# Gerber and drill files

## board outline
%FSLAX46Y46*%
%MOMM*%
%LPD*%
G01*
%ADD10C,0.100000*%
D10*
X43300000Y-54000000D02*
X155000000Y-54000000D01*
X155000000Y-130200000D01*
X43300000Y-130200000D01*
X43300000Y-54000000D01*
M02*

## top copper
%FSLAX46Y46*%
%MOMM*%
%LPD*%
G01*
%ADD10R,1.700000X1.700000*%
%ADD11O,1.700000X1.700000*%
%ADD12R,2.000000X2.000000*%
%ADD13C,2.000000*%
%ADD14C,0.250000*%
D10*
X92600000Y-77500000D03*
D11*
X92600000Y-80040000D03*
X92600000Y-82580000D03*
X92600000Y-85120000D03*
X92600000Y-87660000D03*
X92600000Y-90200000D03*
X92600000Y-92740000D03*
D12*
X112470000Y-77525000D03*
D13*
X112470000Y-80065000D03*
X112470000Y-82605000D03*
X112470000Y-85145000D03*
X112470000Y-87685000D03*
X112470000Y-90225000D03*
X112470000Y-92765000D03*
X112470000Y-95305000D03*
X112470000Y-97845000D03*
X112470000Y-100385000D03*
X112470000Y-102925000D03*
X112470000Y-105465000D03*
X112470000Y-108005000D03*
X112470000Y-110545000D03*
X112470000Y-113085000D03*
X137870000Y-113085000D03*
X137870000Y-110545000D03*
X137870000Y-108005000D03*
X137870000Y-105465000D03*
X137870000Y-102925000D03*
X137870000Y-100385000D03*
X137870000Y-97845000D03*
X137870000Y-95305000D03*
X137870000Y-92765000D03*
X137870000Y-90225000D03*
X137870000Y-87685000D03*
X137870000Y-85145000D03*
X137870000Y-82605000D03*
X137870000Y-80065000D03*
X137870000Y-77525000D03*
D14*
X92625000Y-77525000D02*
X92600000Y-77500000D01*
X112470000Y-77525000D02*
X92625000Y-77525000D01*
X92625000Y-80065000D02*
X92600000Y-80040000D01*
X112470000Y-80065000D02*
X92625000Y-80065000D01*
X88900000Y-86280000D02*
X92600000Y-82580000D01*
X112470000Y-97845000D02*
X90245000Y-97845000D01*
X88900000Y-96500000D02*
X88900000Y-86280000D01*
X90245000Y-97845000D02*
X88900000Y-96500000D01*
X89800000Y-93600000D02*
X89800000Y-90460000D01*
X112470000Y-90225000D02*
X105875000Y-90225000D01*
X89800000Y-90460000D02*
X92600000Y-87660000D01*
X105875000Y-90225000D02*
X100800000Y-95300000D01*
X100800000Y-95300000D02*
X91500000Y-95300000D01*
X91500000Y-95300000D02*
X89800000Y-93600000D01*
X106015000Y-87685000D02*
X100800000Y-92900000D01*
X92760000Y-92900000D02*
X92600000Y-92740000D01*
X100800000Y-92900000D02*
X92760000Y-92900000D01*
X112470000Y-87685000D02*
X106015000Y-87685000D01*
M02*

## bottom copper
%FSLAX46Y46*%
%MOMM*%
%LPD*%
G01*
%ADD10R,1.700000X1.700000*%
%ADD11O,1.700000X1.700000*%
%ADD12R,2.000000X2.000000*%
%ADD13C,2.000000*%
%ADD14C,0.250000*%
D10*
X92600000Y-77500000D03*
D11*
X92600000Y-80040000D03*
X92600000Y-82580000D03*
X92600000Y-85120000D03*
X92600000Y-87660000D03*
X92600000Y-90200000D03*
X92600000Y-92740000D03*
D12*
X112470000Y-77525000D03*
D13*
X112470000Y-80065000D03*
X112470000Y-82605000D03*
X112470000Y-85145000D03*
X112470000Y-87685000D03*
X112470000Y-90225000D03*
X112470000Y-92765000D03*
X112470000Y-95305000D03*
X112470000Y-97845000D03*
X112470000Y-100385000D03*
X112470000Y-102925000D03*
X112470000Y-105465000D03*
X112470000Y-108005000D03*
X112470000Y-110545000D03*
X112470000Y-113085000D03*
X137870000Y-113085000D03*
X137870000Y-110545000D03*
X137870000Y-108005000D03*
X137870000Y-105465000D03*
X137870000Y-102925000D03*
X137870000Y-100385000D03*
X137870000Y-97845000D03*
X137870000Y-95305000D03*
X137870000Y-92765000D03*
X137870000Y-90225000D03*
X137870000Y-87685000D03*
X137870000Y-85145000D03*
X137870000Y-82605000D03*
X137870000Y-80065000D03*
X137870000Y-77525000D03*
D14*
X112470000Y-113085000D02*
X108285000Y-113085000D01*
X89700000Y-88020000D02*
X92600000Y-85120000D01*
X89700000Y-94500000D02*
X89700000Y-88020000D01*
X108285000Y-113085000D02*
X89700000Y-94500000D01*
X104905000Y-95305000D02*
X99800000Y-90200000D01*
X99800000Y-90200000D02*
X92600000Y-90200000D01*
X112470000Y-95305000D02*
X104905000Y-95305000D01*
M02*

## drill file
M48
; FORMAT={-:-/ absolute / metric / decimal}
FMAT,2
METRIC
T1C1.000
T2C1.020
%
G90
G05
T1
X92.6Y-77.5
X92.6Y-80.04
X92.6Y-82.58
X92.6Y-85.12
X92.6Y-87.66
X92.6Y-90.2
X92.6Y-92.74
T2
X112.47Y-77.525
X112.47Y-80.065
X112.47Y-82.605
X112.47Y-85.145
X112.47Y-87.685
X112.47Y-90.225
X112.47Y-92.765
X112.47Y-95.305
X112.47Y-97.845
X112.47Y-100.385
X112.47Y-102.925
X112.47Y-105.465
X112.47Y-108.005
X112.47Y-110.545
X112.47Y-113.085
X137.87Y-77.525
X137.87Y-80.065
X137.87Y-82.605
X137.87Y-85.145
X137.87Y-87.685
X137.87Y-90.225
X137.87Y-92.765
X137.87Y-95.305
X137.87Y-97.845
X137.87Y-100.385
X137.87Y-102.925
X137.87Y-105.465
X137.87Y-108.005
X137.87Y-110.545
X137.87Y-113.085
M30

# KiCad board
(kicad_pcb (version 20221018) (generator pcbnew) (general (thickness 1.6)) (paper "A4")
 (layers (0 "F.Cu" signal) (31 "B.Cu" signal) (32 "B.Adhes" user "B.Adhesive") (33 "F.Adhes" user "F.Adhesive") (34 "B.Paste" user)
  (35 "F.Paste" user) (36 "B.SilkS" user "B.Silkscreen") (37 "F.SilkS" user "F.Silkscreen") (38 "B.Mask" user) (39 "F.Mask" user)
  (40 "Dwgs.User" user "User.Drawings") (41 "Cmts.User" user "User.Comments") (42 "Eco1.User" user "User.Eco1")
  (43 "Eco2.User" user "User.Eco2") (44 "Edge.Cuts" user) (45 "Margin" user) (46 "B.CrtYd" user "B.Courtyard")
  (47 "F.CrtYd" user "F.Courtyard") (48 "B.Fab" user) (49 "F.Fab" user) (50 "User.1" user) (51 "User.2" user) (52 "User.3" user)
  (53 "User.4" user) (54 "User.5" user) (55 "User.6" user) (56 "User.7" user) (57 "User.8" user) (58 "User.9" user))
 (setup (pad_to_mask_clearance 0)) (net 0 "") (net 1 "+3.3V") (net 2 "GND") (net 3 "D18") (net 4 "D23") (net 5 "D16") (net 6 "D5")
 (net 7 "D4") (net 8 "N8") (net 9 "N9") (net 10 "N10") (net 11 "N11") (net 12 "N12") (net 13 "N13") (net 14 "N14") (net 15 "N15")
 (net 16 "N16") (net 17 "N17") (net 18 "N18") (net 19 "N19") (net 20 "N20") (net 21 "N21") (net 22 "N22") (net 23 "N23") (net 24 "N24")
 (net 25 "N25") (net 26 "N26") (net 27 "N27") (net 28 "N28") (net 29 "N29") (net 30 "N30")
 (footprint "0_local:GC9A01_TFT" (layer "F.Cu") (at 92.6 77.5)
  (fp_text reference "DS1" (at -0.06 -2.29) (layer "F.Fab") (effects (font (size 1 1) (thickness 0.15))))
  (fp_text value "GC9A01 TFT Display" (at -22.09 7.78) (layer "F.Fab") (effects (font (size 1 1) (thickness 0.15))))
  (pad "1" thru_hole rect (at 0 0) (size 1.7 1.7) (drill 1) (layers "*.Cu" "*.Mask") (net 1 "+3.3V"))
  (pad "2" thru_hole oval (at 0 2.54) (size 1.7 1.7) (drill 1) (layers "*.Cu" "*.Mask") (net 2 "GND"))
  (pad "3" thru_hole oval (at 0 5.08) (size 1.7 1.7) (drill 1) (layers "*.Cu" "*.Mask") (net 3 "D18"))
  (pad "4" thru_hole oval (at 0 7.62) (size 1.7 1.7) (drill 1) (layers "*.Cu" "*.Mask") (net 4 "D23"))
  (pad "5" thru_hole oval (at 0 10.16) (size 1.7 1.7) (drill 1) (layers "*.Cu" "*.Mask") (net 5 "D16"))
  (pad "6" thru_hole oval (at 0 12.7) (size 1.7 1.7) (drill 1) (layers "*.Cu" "*.Mask") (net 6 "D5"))
  (pad "7" thru_hole oval (at 0 15.24) (size 1.7 1.7) (drill 1) (layers "*.Cu" "*.Mask") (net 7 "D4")))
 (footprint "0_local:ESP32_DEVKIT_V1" (layer "F.Cu") (at 125.17 93.04)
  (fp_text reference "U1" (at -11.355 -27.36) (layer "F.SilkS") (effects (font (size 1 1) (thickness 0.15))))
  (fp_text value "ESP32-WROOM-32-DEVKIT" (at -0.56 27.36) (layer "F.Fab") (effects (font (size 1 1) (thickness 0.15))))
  (pad "1" thru_hole rect (at -12.7 -15.515) (size 2 2) (drill 1.02) (layers "*.Cu" "*.Mask") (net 1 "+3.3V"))
  (pad "2" thru_hole circle (at -12.7 -12.975) (size 2 2) (drill 1.02) (layers "*.Cu" "*.Mask") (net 2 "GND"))
  (pad "3" thru_hole circle (at -12.7 -10.435) (size 2 2) (drill 1.02) (layers "*.Cu" "*.Mask") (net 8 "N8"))
  (pad "4" thru_hole circle (at -12.7 -7.895) (size 2 2) (drill 1.02) (layers "*.Cu" "*.Mask") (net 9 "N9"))
  (pad "5" thru_hole circle (at -12.7 -5.355) (size 2 2) (drill 1.02) (layers "*.Cu" "*.Mask") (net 7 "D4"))
  (pad "6" thru_hole circle (at -12.7 -2.815) (size 2 2) (drill 1.02) (layers "*.Cu" "*.Mask") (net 5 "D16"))
  (pad "7" thru_hole circle (at -12.7 -0.275) (size 2 2) (drill 1.02) (layers "*.Cu" "*.Mask") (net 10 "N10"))
  (pad "8" thru_hole circle (at -12.7 2.265) (size 2 2) (drill 1.02) (layers "*.Cu" "*.Mask") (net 6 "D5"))
  (pad "9" thru_hole circle (at -12.7 4.805) (size 2 2) (drill 1.02) (layers "*.Cu" "*.Mask") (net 3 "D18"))
  (pad "10" thru_hole circle (at -12.7 7.345) (size 2 2) (drill 1.02) (layers "*.Cu" "*.Mask") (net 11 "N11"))
  (pad "11" thru_hole circle (at -12.7 9.885) (size 2 2) (drill 1.02) (layers "*.Cu" "*.Mask") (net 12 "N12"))
  (pad "12" thru_hole circle (at -12.7 12.425) (size 2 2) (drill 1.02) (layers "*.Cu" "*.Mask") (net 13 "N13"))
  (pad "13" thru_hole circle (at -12.7 14.965) (size 2 2) (drill 1.02) (layers "*.Cu" "*.Mask") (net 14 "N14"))
  (pad "14" thru_hole circle (at -12.7 17.505) (size 2 2) (drill 1.02) (layers "*.Cu" "*.Mask") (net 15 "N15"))
  (pad "15" thru_hole circle (at -12.7 20.045) (size 2 2) (drill 1.02) (layers "*.Cu" "*.Mask") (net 4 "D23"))
  (pad "16" thru_hole circle (at 12.7 20.045) (size 2 2) (drill 1.02) (layers "*.Cu" "*.Mask") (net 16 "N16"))
  (pad "17" thru_hole circle (at 12.7 17.505) (size 2 2) (drill 1.02) (layers "*.Cu" "*.Mask") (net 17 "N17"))
  (pad "18" thru_hole circle (at 12.7 14.965) (size 2 2) (drill 1.02) (layers "*.Cu" "*.Mask") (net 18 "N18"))
  (pad "19" thru_hole circle (at 12.7 12.425) (size 2 2) (drill 1.02) (layers "*.Cu" "*.Mask") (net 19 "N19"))
  (pad "20" thru_hole circle (at 12.7 9.885) (size 2 2) (drill 1.02) (layers "*.Cu" "*.Mask") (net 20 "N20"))
  (pad "21" thru_hole circle (at 12.7 7.345) (size 2 2) (drill 1.02) (layers "*.Cu" "*.Mask") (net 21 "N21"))
  (pad "22" thru_hole circle (at 12.7 4.805) (size 2 2) (drill 1.02) (layers "*.Cu" "*.Mask") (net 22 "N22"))
  (pad "23" thru_hole circle (at 12.7 2.265) (size 2 2) (drill 1.02) (layers "*.Cu" "*.Mask") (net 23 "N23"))
  (pad "24" thru_hole circle (at 12.7 -0.275) (size 2 2) (drill 1.02) (layers "*.Cu" "*.Mask") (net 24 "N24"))
  (pad "25" thru_hole circle (at 12.7 -2.815) (size 2 2) (drill 1.02) (layers "*.Cu" "*.Mask") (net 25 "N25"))
  (pad "26" thru_hole circle (at 12.7 -5.355) (size 2 2) (drill 1.02) (layers "*.Cu" "*.Mask") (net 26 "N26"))
  (pad "27" thru_hole circle (at 12.7 -7.895) (size 2 2) (drill 1.02) (layers "*.Cu" "*.Mask") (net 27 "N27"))
  (pad "28" thru_hole circle (at 12.7 -10.435) (size 2 2) (drill 1.02) (layers "*.Cu" "*.Mask") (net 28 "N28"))
  (pad "29" thru_hole circle (at 12.7 -12.975) (size 2 2) (drill 1.02) (layers "*.Cu" "*.Mask") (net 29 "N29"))
  (pad "30" thru_hole circle (at 12.7 -15.515) (size 2 2) (drill 1.02) (layers "*.Cu" "*.Mask") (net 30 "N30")))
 (gr_rect (start 43.3 54) (end 155 130.2) (stroke (width 0.1) (type solid)) (fill none) (layer "Edge.Cuts"))
 (segment (start 92.625 77.525) (end 92.6 77.5) (width 0.25) (layer "F.Cu") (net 1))
 (segment (start 112.47 77.525) (end 92.625 77.525) (width 0.25) (layer "F.Cu") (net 1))
 (segment (start 92.625 80.065) (end 92.6 80.04) (width 0.25) (layer "F.Cu") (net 2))
 (segment (start 112.47 80.065) (end 92.625 80.065) (width 0.25) (layer "F.Cu") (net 2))
 (segment (start 88.9 86.28) (end 92.6 82.58) (width 0.25) (layer "F.Cu") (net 3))
 (segment (start 112.47 97.845) (end 90.245 97.845) (width 0.25) (layer "F.Cu") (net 3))
 (segment (start 88.9 96.5) (end 88.9 86.28) (width 0.25) (layer "F.Cu") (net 3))
 (segment (start 90.245 97.845) (end 88.9 96.5) (width 0.25) (layer "F.Cu") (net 3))
 (segment (start 112.47 113.085) (end 108.285 113.085) (width 0.25) (layer "B.Cu") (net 4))
 (segment (start 89.7 88.02) (end 92.6 85.12) (width 0.25) (layer "B.Cu") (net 4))
 (segment (start 89.7 94.5) (end 89.7 88.02) (width 0.25) (layer "B.Cu") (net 4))
 (segment (start 108.285 113.085) (end 89.7 94.5) (width 0.25) (layer "B.Cu") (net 4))
 (segment (start 89.8 93.6) (end 89.8 90.46) (width 0.25) (layer "F.Cu") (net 5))
 (segment (start 112.47 90.225) (end 105.875 90.225) (width 0.25) (layer "F.Cu") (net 5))
 (segment (start 89.8 90.46) (end 92.6 87.66) (width 0.25) (layer "F.Cu") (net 5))
 (segment (start 105.875 90.225) (end 100.8 95.3) (width 0.25) (layer "F.Cu") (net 5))
 (segment (start 100.8 95.3) (end 91.5 95.3) (width 0.25) (layer "F.Cu") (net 5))
 (segment (start 91.5 95.3) (end 89.8 93.6) (width 0.25) (layer "F.Cu") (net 5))
 (segment (start 104.905 95.305) (end 99.8 90.2) (width 0.25) (layer "B.Cu") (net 6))
 (segment (start 99.8 90.2) (end 92.6 90.2) (width 0.25) (layer "B.Cu") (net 6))
 (segment (start 112.47 95.305) (end 104.905 95.305) (width 0.25) (layer "B.Cu") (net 6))
 (segment (start 106.015 87.685) (end 100.8 92.9) (width 0.25) (layer "F.Cu") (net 7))
 (segment (start 92.76 92.9) (end 92.6 92.74) (width 0.25) (layer "F.Cu") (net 7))
 (segment (start 100.8 92.9) (end 92.76 92.9) (width 0.25) (layer "F.Cu") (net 7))
 (segment (start 112.47 87.685) (end 106.015 87.685) (width 0.25) (layer "F.Cu") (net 7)))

